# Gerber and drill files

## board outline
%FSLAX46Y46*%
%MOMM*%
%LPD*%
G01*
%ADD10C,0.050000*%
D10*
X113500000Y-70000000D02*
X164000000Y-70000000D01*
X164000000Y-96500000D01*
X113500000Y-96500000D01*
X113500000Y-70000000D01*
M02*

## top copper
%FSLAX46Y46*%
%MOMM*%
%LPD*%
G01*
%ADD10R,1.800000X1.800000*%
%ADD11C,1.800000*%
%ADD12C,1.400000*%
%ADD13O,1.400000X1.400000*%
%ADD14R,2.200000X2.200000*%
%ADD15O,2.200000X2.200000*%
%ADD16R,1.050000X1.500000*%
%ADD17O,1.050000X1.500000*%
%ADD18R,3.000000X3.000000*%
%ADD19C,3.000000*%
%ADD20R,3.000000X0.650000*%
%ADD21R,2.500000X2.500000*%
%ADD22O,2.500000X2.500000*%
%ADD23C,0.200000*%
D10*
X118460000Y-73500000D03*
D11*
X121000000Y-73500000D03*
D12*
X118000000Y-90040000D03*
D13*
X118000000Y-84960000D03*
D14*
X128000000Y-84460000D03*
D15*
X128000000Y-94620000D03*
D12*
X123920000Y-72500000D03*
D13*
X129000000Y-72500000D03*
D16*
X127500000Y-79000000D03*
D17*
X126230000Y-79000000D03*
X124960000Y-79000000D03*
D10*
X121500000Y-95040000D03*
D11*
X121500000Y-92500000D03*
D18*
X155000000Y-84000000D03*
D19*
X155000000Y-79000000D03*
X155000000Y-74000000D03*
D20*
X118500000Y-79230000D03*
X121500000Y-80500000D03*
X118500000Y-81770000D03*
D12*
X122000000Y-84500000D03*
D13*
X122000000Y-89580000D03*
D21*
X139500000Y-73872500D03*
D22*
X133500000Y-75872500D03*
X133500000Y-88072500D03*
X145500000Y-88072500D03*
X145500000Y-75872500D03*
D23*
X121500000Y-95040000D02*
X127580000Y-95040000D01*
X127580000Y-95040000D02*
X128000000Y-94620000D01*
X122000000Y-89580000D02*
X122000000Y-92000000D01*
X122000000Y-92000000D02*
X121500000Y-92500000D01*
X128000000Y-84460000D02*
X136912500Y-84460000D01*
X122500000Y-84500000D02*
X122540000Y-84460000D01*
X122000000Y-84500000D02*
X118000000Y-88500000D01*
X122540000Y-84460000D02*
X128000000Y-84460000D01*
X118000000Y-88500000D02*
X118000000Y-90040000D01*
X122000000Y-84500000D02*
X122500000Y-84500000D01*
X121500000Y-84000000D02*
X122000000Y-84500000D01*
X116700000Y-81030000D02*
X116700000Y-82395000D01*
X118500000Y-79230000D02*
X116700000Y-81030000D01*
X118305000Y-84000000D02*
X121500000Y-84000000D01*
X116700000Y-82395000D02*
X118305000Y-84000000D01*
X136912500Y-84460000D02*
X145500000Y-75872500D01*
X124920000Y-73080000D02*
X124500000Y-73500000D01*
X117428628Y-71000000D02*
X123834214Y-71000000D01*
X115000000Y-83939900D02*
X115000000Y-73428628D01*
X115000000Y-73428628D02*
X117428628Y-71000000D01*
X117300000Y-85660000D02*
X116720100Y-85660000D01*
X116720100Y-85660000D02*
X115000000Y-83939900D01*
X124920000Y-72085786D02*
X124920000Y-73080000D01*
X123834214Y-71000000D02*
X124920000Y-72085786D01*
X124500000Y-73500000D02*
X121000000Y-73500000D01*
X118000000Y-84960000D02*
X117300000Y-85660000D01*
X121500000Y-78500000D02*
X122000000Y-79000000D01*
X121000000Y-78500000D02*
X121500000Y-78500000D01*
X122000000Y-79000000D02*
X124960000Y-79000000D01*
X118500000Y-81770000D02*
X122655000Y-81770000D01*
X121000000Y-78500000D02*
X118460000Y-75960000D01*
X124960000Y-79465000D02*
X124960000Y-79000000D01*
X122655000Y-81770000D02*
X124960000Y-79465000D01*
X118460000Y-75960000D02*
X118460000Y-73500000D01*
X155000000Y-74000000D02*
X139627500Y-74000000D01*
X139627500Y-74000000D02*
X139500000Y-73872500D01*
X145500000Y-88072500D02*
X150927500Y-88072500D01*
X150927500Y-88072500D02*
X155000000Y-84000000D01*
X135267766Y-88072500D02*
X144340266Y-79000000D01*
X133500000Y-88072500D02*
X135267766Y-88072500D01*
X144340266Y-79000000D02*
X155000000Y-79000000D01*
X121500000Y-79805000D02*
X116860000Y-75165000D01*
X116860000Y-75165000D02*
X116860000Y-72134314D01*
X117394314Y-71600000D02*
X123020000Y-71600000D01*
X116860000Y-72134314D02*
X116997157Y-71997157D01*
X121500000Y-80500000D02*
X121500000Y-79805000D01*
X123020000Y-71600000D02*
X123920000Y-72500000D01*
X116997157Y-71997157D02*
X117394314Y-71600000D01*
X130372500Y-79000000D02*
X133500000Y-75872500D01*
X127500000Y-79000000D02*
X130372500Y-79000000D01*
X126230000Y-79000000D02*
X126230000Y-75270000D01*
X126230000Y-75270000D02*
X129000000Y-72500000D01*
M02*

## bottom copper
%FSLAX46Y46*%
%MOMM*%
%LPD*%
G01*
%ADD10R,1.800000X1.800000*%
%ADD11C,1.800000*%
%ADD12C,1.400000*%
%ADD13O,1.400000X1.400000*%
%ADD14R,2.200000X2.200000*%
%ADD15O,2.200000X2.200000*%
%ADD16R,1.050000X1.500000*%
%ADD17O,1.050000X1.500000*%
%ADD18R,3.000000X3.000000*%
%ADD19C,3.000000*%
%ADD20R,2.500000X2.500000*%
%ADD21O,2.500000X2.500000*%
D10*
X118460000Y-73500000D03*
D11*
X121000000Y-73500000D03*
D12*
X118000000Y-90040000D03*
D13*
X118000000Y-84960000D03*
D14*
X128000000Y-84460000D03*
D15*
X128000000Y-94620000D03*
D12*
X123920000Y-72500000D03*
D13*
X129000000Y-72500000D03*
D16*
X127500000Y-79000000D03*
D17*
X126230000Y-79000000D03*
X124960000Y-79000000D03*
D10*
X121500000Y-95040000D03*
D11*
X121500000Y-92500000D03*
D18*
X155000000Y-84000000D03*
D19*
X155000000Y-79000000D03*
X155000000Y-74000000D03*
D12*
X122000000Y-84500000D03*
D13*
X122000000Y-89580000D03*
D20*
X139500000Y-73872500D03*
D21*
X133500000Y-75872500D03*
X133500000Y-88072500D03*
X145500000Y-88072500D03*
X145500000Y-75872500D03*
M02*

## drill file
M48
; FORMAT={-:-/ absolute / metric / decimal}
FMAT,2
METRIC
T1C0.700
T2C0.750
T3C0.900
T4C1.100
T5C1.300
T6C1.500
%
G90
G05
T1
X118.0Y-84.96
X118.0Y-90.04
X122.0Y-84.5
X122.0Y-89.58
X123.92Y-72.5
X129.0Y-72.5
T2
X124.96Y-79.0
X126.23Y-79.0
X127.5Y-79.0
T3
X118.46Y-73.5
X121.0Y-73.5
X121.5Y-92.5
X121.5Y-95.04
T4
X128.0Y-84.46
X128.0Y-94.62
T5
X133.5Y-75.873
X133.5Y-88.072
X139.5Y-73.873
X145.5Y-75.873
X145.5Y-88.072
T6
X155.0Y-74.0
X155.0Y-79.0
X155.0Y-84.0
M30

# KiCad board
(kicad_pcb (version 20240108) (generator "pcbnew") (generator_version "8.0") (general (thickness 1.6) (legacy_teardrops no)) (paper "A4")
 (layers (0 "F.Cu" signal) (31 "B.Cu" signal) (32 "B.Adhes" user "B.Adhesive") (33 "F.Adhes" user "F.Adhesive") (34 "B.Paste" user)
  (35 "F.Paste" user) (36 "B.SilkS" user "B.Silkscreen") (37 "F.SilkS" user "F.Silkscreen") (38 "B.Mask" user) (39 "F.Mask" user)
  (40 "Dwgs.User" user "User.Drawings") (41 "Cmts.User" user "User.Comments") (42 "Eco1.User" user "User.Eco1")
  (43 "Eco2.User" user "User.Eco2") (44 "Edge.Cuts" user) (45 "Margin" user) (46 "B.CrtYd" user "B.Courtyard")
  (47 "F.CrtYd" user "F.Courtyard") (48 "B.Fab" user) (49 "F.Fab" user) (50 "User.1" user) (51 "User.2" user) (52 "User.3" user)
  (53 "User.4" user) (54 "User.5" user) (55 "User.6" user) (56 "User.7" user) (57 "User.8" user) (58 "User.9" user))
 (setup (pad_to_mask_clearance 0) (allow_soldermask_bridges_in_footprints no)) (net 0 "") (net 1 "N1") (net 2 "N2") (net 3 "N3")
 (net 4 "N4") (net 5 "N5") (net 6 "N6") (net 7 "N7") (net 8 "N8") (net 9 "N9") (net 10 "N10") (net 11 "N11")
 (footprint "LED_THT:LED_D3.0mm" (layer "F.Cu") (at 118.46 73.5)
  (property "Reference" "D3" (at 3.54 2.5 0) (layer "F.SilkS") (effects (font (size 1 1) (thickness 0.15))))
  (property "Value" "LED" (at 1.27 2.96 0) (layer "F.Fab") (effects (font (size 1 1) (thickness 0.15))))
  (pad "1" thru_hole rect (at 0 0) (size 1.8 1.8) (drill 0.9) (layers "*.Cu" "*.Mask") (remove_unused_layers no) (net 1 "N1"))
  (pad "2" thru_hole circle (at 2.54 0) (size 1.8 1.8) (drill 0.9) (layers "*.Cu" "*.Mask") (remove_unused_layers no) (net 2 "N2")))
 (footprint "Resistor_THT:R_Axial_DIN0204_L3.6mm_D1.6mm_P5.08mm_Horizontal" (layer "F.Cu") (at 118 90.04 90)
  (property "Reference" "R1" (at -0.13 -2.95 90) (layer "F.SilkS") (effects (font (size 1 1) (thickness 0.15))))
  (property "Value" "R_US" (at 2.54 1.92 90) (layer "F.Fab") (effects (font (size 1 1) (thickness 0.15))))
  (pad "1" thru_hole circle (at 0 0 90) (size 1.4 1.4) (drill 0.7) (layers "*.Cu" "*.Mask") (remove_unused_layers no) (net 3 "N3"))
  (pad "2" thru_hole oval (at 5.08 0 90) (size 1.4 1.4) (drill 0.7) (layers "*.Cu" "*.Mask") (remove_unused_layers no) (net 2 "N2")))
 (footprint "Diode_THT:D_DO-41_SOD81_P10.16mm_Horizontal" (layer "F.Cu") (at 128 84.46 -90)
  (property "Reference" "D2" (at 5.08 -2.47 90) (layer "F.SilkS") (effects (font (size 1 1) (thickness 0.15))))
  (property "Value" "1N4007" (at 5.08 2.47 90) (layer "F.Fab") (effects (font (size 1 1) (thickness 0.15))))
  (pad "1" thru_hole rect (at 0 0 270) (size 2.2 2.2) (drill 1.1) (layers "*.Cu" "*.Mask") (remove_unused_layers no) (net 3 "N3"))
  (pad "2" thru_hole oval (at 10.16 0 270) (size 2.2 2.2) (drill 1.1) (layers "*.Cu" "*.Mask") (remove_unused_layers no) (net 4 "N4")))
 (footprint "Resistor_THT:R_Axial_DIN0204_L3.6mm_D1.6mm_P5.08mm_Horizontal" (layer "F.Cu") (at 123.92 72.5)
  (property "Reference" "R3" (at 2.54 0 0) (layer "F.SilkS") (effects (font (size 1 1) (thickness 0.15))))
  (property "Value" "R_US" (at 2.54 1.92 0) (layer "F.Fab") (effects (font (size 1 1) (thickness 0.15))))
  (pad "1" thru_hole circle (at 0 0) (size 1.4 1.4) (drill 0.7) (layers "*.Cu" "*.Mask") (remove_unused_layers no) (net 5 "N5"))
  (pad "2" thru_hole oval (at 5.08 0) (size 1.4 1.4) (drill 0.7) (layers "*.Cu" "*.Mask") (remove_unused_layers no) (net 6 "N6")))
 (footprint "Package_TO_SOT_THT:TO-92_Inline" (layer "F.Cu") (at 127.5 79 180)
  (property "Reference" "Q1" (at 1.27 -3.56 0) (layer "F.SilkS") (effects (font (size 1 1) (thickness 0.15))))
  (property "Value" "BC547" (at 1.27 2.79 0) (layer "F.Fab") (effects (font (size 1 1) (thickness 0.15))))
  (pad "1" thru_hole rect (at 0 0 180) (size 1.05 1.5) (drill 0.75) (layers "*.Cu" "*.Mask") (remove_unused_layers no) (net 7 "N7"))
  (pad "2" thru_hole oval (at 1.27 0 180) (size 1.05 1.5) (drill 0.75) (layers "*.Cu" "*.Mask") (remove_unused_layers no) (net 6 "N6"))
  (pad "3" thru_hole oval (at 2.54 0 180) (size 1.05 1.5) (drill 0.75) (layers "*.Cu" "*.Mask") (remove_unused_layers no) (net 1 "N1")))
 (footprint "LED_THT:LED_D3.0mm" (layer "F.Cu") (at 121.5 95.04 90)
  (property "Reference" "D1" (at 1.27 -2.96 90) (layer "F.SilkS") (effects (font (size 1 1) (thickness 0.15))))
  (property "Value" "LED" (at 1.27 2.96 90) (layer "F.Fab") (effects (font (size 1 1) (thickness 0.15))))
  (pad "1" thru_hole rect (at 0 0 90) (size 1.8 1.8) (drill 0.9) (layers "*.Cu" "*.Mask") (remove_unused_layers no) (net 4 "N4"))
  (pad "2" thru_hole circle (at 2.54 0 90) (size 1.8 1.8) (drill 0.9) (layers "*.Cu" "*.Mask") (remove_unused_layers no) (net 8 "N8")))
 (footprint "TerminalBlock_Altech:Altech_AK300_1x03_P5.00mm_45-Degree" (layer "F.Cu") (at 155 84 90)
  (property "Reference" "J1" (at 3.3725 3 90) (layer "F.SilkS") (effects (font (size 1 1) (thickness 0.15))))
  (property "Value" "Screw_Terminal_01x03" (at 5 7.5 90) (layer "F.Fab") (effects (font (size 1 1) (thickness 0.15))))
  (pad "1" thru_hole rect (at 0 0 90) (size 3 3) (drill 1.5) (layers "*.Cu" "*.Mask") (remove_unused_layers no) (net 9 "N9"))
  (pad "2" thru_hole circle (at 5 0 90) (size 3 3) (drill 1.5) (layers "*.Cu" "*.Mask") (remove_unused_layers no) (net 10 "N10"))
  (pad "3" thru_hole circle (at 10 0 90) (size 3 3) (drill 1.5) (layers "*.Cu" "*.Mask") (remove_unused_layers no) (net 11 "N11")))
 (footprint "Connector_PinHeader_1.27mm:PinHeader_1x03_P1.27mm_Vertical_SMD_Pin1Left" (layer "F.Cu") (at 120 80.5)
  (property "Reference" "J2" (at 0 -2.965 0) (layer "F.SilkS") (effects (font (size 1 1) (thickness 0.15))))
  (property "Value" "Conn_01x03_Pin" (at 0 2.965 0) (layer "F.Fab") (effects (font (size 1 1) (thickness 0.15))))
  (pad "1" smd rect (at -1.5 -1.27) (size 3 0.65) (layers "F.Cu" "F.Paste" "F.Mask") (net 3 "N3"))
  (pad "2" smd rect (at 1.5 0) (size 3 0.65) (layers "F.Cu" "F.Paste" "F.Mask") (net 5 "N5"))
  (pad "3" smd rect (at -1.5 1.27) (size 3 0.65) (layers "F.Cu" "F.Paste" "F.Mask") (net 1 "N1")))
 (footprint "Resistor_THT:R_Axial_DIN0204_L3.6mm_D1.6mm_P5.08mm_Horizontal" (layer "F.Cu") (at 122 84.5 -90)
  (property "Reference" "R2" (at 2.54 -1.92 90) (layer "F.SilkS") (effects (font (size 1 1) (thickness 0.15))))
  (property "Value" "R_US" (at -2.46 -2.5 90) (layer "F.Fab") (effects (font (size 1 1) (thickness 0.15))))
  (pad "1" thru_hole circle (at 0 0 270) (size 1.4 1.4) (drill 0.7) (layers "*.Cu" "*.Mask") (remove_unused_layers no) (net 3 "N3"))
  (pad "2" thru_hole oval (at 5.08 0 270) (size 1.4 1.4) (drill 0.7) (layers "*.Cu" "*.Mask") (remove_unused_layers no) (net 8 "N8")))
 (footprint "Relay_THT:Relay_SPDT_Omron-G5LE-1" (layer "F.Cu") (at 139.5 73.8725)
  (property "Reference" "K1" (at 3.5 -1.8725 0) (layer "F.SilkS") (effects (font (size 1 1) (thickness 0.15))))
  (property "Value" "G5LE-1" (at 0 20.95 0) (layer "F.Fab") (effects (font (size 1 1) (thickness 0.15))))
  (pad "1" thru_hole rect (at 0 0) (size 2.5 2.5) (drill 1.3) (layers "*.Cu" "*.Mask") (remove_unused_layers no) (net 11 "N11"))
  (pad "2" thru_hole oval (at -6 2) (size 2.5 2.5) (drill 1.3) (layers "*.Cu" "*.Mask") (remove_unused_layers no) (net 7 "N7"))
  (pad "3" thru_hole oval (at -6 14.2) (size 2.5 2.5) (drill 1.3) (layers "*.Cu" "*.Mask") (remove_unused_layers no) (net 10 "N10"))
  (pad "4" thru_hole oval (at 6 14.2) (size 2.5 2.5) (drill 1.3) (layers "*.Cu" "*.Mask") (remove_unused_layers no) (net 9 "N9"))
  (pad "5" thru_hole oval (at 6 2) (size 2.5 2.5) (drill 1.3) (layers "*.Cu" "*.Mask") (remove_unused_layers no) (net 3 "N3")))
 (gr_rect (start 113.5 70) (end 164 96.5) (stroke (width 0.05) (type default)) (fill none) (layer "Edge.Cuts"))
 (segment (start 121.5 95.04) (end 127.58 95.04) (width 0.2) (layer "F.Cu") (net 4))
 (segment (start 127.58 95.04) (end 128 94.62) (width 0.2) (layer "F.Cu") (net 4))
 (segment (start 122 89.58) (end 122 92) (width 0.2) (layer "F.Cu") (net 8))
 (segment (start 122 92) (end 121.5 92.5) (width 0.2) (layer "F.Cu") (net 8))
 (segment (start 128 84.46) (end 136.9125 84.46) (width 0.2) (layer "F.Cu") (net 3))
 (segment (start 122.5 84.5) (end 122.54 84.46) (width 0.2) (layer "F.Cu") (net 3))
 (segment (start 122 84.5) (end 118 88.5) (width 0.2) (layer "F.Cu") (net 3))
 (segment (start 122.54 84.46) (end 128 84.46) (width 0.2) (layer "F.Cu") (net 3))
 (segment (start 118 88.5) (end 118 90.04) (width 0.2) (layer "F.Cu") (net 3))
 (segment (start 122 84.5) (end 122.5 84.5) (width 0.2) (layer "F.Cu") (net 3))
 (segment (start 121.5 84) (end 122 84.5) (width 0.2) (layer "F.Cu") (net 3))
 (segment (start 116.7 81.03) (end 116.7 82.395) (width 0.2) (layer "F.Cu") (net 3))
 (segment (start 118.5 79.23) (end 116.7 81.03) (width 0.2) (layer "F.Cu") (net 3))
 (segment (start 118.305 84) (end 121.5 84) (width 0.2) (layer "F.Cu") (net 3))
 (segment (start 116.7 82.395) (end 118.305 84) (width 0.2) (layer "F.Cu") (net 3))
 (segment (start 136.9125 84.46) (end 145.5 75.8725) (width 0.2) (layer "F.Cu") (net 3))
 (segment (start 124.92 73.08) (end 124.5 73.5) (width 0.2) (layer "F.Cu") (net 2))
 (segment (start 117.428628 71) (end 123.834214 71) (width 0.2) (layer "F.Cu") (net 2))
 (segment (start 115 83.9399) (end 115 73.428628) (width 0.2) (layer "F.Cu") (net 2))
 (segment (start 115 73.428628) (end 117.428628 71) (width 0.2) (layer "F.Cu") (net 2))
 (segment (start 117.3 85.66) (end 116.7201 85.66) (width 0.2) (layer "F.Cu") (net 2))
 (segment (start 116.7201 85.66) (end 115 83.9399) (width 0.2) (layer "F.Cu") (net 2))
 (segment (start 124.92 72.085786) (end 124.92 73.08) (width 0.2) (layer "F.Cu") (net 2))
 (segment (start 123.834214 71) (end 124.92 72.085786) (width 0.2) (layer "F.Cu") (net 2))
 (segment (start 124.5 73.5) (end 121 73.5) (width 0.2) (layer "F.Cu") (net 2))
 (segment (start 118 84.96) (end 117.3 85.66) (width 0.2) (layer "F.Cu") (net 2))
 (segment (start 121.5 78.5) (end 122 79) (width 0.2) (layer "F.Cu") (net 1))
 (segment (start 121 78.5) (end 121.5 78.5) (width 0.2) (layer "F.Cu") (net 1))
 (segment (start 122 79) (end 124.96 79) (width 0.2) (layer "F.Cu") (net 1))
 (segment (start 118.5 81.77) (end 122.655 81.77) (width 0.2) (layer "F.Cu") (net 1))
 (segment (start 121 78.5) (end 118.46 75.96) (width 0.2) (layer "F.Cu") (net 1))
 (segment (start 124.96 79.465) (end 124.96 79) (width 0.2) (layer "F.Cu") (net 1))
 (segment (start 122.655 81.77) (end 124.96 79.465) (width 0.2) (layer "F.Cu") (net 1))
 (segment (start 118.46 75.96) (end 118.46 73.5) (width 0.2) (layer "F.Cu") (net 1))
 (segment (start 155 74) (end 139.6275 74) (width 0.2) (layer "F.Cu") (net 11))
 (segment (start 139.6275 74) (end 139.5 73.8725) (width 0.2) (layer "F.Cu") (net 11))
 (segment (start 145.5 88.0725) (end 150.9275 88.0725) (width 0.2) (layer "F.Cu") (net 9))
 (segment (start 150.9275 88.0725) (end 155 84) (width 0.2) (layer "F.Cu") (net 9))
 (segment (start 135.267766 88.0725) (end 144.340266 79) (width 0.2) (layer "F.Cu") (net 10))
 (segment (start 133.5 88.0725) (end 135.267766 88.0725) (width 0.2) (layer "F.Cu") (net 10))
 (segment (start 144.340266 79) (end 155 79) (width 0.2) (layer "F.Cu") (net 10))
 (segment (start 121.5 79.805) (end 116.86 75.165) (width 0.2) (layer "F.Cu") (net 5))
 (segment (start 116.86 75.165) (end 116.86 72.134314) (width 0.2) (layer "F.Cu") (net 5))
 (segment (start 117.394314 71.6) (end 123.02 71.6) (width 0.2) (layer "F.Cu") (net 5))
 (segment (start 116.86 72.134314) (end 116.997157 71.997157) (width 0.2) (layer "F.Cu") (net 5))
 (segment (start 121.5 80.5) (end 121.5 79.805) (width 0.2) (layer "F.Cu") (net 5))
 (segment (start 123.02 71.6) (end 123.92 72.5) (width 0.2) (layer "F.Cu") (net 5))
 (segment (start 116.997157 71.997157) (end 117.394314 71.6) (width 0.2) (layer "F.Cu") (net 5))
 (segment (start 130.3725 79) (end 133.5 75.8725) (width 0.2) (layer "F.Cu") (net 7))
 (segment (start 127.5 79) (end 130.3725 79) (width 0.2) (layer "F.Cu") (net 7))
 (segment (start 126.23 79) (end 126.23 75.27) (width 0.2) (layer "F.Cu") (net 6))
 (segment (start 126.23 75.27) (end 129 72.5) (width 0.2) (layer "F.Cu") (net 6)))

